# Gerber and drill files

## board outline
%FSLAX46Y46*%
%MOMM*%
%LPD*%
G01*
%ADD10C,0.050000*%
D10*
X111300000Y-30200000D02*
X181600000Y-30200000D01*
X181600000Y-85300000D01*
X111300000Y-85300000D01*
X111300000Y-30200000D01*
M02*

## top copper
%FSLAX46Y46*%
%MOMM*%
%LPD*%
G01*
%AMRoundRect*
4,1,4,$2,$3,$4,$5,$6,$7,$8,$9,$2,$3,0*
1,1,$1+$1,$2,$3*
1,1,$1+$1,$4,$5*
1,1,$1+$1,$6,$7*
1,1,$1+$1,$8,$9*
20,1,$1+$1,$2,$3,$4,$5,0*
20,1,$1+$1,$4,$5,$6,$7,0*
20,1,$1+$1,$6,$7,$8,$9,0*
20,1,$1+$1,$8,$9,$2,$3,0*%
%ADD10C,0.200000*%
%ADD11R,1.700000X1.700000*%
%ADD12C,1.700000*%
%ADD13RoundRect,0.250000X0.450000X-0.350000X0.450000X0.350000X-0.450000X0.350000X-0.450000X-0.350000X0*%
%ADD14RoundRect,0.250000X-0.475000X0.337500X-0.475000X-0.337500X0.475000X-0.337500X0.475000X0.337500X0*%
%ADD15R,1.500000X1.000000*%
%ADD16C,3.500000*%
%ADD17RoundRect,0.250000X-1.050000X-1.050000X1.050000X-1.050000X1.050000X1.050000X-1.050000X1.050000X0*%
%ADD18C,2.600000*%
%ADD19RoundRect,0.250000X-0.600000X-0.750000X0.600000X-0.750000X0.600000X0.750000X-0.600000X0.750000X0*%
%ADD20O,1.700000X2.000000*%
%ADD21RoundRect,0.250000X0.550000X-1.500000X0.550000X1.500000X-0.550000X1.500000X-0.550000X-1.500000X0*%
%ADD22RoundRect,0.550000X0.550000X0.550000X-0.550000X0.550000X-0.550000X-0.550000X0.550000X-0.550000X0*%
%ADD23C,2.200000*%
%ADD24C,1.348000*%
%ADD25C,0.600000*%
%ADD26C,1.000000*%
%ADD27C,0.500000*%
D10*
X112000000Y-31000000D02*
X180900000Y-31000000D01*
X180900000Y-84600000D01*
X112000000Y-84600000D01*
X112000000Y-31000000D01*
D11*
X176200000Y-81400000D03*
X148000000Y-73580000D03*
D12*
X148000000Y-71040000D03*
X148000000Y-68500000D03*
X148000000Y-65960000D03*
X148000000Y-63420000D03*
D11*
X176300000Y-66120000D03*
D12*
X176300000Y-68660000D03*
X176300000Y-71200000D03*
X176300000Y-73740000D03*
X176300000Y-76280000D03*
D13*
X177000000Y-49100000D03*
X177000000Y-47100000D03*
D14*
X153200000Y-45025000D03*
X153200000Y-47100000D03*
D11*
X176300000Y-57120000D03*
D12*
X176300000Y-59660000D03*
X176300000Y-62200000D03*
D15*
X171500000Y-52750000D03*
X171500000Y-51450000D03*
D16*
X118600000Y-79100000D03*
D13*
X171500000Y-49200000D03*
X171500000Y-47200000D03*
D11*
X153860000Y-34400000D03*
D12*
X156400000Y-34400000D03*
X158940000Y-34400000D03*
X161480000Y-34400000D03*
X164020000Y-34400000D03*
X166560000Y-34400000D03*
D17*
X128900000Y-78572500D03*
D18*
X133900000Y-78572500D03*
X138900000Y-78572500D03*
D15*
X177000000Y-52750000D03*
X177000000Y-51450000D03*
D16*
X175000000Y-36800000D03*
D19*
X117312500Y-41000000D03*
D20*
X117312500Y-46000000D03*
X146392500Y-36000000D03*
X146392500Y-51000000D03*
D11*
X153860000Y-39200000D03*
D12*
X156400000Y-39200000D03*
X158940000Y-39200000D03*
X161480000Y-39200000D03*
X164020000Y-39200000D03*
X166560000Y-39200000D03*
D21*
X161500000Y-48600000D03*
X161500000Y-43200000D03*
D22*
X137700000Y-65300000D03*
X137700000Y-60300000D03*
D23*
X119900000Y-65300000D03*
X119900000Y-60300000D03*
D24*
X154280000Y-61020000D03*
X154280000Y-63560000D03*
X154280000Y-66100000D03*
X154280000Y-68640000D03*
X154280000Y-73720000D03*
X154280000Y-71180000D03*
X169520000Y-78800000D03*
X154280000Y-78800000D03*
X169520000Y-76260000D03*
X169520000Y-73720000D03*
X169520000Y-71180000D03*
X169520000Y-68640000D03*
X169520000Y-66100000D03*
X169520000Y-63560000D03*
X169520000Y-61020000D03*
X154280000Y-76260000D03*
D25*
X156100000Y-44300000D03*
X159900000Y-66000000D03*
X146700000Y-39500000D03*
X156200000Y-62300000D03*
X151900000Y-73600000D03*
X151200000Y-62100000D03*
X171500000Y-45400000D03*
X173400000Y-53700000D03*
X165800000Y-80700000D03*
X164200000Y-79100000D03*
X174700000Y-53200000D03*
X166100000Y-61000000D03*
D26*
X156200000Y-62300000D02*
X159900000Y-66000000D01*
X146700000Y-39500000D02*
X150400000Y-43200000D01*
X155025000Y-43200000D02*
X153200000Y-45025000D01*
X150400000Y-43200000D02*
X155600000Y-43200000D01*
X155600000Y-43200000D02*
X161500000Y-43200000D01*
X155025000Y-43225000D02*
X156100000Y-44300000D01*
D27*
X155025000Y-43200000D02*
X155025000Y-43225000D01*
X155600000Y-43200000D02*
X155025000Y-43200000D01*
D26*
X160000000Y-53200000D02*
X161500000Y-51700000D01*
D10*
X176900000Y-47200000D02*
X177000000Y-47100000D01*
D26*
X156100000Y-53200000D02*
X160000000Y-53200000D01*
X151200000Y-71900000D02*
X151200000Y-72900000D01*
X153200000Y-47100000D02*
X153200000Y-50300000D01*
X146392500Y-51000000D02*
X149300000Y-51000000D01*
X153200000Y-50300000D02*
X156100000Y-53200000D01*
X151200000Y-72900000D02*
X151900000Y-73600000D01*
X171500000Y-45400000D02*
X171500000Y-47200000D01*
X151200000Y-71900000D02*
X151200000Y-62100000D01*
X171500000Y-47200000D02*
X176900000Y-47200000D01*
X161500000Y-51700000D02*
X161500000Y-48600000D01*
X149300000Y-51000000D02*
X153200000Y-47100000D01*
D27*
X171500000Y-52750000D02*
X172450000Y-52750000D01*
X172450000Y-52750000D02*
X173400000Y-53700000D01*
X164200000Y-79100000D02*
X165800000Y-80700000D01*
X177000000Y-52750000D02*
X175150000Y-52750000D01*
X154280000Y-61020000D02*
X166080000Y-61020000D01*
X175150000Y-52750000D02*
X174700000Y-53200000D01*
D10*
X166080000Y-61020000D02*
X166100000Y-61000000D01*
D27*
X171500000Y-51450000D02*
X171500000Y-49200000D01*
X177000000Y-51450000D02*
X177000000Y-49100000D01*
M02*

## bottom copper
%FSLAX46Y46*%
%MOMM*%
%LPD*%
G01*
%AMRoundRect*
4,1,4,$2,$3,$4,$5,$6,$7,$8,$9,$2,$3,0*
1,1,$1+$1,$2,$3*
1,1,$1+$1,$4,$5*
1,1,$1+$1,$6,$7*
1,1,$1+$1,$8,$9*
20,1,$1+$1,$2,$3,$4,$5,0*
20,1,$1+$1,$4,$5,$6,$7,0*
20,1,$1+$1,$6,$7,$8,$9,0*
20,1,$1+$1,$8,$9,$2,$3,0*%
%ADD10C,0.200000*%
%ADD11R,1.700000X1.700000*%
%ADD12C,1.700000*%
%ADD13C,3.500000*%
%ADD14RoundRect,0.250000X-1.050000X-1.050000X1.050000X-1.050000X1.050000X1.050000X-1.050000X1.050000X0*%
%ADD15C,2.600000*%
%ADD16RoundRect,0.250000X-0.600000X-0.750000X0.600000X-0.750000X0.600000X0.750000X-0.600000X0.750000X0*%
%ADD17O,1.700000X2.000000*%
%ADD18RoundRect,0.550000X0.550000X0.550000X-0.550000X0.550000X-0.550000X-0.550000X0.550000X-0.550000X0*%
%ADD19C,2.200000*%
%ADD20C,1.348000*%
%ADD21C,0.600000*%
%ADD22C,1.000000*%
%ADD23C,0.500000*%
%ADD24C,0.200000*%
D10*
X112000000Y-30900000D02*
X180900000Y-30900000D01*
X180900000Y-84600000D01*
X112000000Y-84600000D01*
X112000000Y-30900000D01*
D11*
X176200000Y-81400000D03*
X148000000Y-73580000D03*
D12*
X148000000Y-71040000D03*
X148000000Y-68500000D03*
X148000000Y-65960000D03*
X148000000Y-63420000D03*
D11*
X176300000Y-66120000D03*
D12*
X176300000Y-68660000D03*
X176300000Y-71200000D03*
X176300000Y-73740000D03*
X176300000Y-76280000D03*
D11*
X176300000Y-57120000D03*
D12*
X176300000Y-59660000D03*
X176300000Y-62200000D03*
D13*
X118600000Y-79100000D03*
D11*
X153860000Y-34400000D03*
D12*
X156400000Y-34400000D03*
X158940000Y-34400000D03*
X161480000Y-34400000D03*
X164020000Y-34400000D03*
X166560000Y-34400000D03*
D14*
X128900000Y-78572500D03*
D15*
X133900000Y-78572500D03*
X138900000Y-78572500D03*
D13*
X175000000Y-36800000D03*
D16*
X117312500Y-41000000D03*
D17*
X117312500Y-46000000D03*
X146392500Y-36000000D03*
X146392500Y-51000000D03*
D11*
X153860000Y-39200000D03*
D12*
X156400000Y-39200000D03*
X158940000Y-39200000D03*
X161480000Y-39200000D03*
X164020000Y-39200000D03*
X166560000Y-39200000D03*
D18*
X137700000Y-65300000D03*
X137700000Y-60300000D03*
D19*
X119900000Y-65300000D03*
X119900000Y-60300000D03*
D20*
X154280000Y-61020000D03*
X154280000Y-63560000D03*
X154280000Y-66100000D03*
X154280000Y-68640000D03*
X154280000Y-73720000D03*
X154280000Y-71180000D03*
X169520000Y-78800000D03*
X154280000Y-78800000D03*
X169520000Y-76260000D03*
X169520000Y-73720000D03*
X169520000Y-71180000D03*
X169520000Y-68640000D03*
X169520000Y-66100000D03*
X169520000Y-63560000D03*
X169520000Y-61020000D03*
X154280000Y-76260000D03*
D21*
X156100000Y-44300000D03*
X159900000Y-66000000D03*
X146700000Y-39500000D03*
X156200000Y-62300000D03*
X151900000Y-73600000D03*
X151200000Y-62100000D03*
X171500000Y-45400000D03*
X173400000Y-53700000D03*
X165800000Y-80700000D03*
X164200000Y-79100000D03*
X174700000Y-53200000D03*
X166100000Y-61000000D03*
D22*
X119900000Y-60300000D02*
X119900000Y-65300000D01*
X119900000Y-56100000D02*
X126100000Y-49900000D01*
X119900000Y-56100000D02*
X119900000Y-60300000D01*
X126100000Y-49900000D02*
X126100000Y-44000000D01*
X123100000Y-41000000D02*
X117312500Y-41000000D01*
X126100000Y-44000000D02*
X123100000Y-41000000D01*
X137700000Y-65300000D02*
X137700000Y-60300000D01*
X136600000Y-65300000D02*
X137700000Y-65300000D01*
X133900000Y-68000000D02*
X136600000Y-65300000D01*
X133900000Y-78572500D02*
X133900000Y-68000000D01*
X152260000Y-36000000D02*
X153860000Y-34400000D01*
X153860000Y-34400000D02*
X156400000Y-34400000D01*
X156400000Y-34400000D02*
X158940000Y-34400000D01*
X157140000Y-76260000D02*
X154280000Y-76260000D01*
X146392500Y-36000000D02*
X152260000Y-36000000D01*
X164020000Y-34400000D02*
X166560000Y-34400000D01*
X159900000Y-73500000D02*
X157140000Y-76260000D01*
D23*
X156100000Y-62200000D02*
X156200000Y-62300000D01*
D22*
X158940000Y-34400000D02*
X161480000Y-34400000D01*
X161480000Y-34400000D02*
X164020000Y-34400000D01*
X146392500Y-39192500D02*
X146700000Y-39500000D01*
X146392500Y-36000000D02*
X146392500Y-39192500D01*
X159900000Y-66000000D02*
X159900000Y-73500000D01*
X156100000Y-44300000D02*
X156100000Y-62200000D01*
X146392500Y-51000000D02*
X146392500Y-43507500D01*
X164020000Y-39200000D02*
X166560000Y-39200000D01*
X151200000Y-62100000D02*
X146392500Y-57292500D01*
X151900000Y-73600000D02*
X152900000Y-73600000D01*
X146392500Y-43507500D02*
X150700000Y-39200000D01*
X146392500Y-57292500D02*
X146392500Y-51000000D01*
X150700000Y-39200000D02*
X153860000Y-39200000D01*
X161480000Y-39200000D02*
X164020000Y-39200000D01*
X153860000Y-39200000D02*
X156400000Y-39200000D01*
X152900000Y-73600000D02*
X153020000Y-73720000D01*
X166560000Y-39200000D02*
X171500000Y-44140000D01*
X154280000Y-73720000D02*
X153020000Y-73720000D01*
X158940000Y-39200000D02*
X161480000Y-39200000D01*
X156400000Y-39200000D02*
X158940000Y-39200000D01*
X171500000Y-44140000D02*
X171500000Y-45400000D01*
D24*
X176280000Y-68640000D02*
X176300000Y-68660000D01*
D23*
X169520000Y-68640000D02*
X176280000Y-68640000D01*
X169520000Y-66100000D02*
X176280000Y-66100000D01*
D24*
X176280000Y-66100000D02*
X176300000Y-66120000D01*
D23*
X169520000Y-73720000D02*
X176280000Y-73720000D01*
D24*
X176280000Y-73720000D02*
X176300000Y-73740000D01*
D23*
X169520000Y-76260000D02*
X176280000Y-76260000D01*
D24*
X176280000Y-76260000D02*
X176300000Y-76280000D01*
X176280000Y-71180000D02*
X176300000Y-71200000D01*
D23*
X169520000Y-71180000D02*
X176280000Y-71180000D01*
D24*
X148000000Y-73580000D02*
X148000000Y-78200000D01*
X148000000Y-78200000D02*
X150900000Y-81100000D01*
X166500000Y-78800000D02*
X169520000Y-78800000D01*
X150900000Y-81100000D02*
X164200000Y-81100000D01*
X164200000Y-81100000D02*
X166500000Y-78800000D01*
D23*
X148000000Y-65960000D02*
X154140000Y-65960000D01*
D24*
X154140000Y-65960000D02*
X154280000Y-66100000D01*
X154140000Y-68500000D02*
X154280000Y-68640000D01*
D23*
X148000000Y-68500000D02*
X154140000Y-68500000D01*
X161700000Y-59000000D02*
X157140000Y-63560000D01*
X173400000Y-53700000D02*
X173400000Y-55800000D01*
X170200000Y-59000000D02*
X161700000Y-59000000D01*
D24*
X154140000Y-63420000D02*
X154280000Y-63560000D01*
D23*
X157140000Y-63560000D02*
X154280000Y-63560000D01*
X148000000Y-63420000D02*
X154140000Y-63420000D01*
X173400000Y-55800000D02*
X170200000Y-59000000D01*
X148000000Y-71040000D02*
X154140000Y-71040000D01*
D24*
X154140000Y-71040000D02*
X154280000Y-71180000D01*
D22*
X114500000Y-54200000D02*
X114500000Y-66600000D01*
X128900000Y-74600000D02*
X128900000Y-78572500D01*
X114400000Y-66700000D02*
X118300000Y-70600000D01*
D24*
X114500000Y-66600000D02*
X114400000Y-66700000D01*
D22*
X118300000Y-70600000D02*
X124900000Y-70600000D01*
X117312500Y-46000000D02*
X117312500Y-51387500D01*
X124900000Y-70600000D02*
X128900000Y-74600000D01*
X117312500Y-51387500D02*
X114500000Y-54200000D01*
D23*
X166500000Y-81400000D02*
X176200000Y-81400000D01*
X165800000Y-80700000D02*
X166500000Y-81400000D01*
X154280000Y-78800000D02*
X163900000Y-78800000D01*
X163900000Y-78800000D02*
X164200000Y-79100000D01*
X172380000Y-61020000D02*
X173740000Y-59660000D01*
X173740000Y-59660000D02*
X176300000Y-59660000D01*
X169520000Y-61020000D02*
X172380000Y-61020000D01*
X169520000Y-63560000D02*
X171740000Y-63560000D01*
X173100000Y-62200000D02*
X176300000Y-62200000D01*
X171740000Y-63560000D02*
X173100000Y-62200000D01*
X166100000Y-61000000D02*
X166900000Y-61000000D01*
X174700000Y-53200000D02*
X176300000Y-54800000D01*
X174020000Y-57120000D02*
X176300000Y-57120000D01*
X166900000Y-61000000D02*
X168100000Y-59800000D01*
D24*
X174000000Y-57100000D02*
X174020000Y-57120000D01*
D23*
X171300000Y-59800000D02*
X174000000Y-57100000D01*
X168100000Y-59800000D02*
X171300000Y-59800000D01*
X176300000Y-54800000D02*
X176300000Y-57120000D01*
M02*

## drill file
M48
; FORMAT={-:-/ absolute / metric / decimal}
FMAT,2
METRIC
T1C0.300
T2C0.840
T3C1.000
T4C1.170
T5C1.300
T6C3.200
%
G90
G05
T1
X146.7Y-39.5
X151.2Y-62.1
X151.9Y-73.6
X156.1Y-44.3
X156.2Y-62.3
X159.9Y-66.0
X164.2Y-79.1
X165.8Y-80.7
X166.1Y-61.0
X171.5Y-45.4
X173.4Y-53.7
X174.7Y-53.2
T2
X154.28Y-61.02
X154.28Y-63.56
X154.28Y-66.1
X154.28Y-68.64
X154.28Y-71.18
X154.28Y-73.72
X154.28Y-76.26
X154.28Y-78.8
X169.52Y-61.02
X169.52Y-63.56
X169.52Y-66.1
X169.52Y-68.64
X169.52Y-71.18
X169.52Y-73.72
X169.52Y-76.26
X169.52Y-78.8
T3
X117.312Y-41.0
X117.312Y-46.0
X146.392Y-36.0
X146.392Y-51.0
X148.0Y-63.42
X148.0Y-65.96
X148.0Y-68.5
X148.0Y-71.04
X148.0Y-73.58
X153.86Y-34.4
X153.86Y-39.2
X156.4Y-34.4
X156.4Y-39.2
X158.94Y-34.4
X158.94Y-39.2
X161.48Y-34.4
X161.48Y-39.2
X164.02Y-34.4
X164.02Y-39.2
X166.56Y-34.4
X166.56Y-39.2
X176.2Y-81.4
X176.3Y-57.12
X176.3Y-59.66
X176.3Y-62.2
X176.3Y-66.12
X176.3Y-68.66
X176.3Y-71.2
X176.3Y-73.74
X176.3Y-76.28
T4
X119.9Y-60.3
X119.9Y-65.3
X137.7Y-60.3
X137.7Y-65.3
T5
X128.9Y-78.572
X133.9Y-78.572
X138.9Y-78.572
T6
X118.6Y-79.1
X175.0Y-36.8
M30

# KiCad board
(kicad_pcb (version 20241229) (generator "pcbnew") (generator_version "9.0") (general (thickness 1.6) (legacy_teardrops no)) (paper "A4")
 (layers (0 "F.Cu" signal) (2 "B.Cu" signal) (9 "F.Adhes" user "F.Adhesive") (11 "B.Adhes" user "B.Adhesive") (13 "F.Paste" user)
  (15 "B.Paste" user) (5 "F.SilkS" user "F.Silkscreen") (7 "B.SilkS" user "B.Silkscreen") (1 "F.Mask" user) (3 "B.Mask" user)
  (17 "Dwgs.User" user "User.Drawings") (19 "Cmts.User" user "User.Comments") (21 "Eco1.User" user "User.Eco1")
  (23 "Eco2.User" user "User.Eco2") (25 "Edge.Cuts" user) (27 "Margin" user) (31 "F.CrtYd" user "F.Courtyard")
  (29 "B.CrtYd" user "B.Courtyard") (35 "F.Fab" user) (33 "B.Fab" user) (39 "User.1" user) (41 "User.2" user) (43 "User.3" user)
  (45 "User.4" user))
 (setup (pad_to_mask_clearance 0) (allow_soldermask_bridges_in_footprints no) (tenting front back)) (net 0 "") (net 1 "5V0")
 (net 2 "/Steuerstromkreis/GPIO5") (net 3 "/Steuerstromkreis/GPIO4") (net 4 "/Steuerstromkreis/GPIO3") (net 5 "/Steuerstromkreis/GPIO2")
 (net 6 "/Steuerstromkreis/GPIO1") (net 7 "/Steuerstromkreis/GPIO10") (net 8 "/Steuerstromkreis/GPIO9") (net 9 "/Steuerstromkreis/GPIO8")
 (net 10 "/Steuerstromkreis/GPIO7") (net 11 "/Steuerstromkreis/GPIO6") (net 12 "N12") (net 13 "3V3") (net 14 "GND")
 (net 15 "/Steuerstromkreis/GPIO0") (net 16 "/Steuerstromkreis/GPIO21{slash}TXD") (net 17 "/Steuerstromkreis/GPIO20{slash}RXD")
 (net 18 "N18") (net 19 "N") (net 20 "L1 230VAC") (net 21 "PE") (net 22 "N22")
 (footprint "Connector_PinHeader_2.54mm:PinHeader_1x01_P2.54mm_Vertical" (layer "F.Cu") (at 176.2 81.4)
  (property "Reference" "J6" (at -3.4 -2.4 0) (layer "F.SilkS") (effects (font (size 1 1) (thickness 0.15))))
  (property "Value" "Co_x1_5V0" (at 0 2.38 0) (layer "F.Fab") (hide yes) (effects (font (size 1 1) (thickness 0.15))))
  (pad "1" thru_hole rect (at 0 0) (size 1.7 1.7) (drill 1) (layers "*.Cu" "*.Mask") (remove_unused_layers no) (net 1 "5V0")))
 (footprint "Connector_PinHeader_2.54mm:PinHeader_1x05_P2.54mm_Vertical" (layer "F.Cu") (at 148 73.58 180)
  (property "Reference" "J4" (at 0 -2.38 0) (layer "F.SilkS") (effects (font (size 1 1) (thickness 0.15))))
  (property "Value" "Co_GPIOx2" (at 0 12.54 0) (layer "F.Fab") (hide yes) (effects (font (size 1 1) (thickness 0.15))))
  (pad "1" thru_hole rect (at 0 0 180) (size 1.7 1.7) (drill 1) (layers "*.Cu" "*.Mask") (remove_unused_layers no)
   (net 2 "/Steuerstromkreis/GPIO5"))
  (pad "2" thru_hole circle (at 0 2.54 180) (size 1.7 1.7) (drill 1) (layers "*.Cu" "*.Mask") (remove_unused_layers no)
   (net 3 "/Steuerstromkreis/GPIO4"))
  (pad "3" thru_hole circle (at 0 5.08 180) (size 1.7 1.7) (drill 1) (layers "*.Cu" "*.Mask") (remove_unused_layers no)
   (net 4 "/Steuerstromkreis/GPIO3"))
  (pad "4" thru_hole circle (at 0 7.62 180) (size 1.7 1.7) (drill 1) (layers "*.Cu" "*.Mask") (remove_unused_layers no)
   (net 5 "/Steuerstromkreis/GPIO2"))
  (pad "5" thru_hole circle (at 0 10.16 180) (size 1.7 1.7) (drill 1) (layers "*.Cu" "*.Mask") (remove_unused_layers no)
   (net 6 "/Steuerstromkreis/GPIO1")))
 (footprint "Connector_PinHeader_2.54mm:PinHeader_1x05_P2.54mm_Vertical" (layer "F.Cu") (at 176.3 66.12)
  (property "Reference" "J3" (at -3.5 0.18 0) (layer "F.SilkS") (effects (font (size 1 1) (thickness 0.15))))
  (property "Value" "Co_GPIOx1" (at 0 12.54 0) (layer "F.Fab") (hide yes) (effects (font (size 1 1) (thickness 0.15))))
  (pad "1" thru_hole rect (at 0 0) (size 1.7 1.7) (drill 1) (layers "*.Cu" "*.Mask") (remove_unused_layers no)
   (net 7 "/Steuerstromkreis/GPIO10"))
  (pad "2" thru_hole circle (at 0 2.54) (size 1.7 1.7) (drill 1) (layers "*.Cu" "*.Mask") (remove_unused_layers no)
   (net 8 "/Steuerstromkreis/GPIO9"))
  (pad "3" thru_hole circle (at 0 5.08) (size 1.7 1.7) (drill 1) (layers "*.Cu" "*.Mask") (remove_unused_layers no)
   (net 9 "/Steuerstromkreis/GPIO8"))
  (pad "4" thru_hole circle (at 0 7.62) (size 1.7 1.7) (drill 1) (layers "*.Cu" "*.Mask") (remove_unused_layers no)
   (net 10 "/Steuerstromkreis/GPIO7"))
  (pad "5" thru_hole circle (at 0 10.16) (size 1.7 1.7) (drill 1) (layers "*.Cu" "*.Mask") (remove_unused_layers no)
   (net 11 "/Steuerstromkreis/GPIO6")))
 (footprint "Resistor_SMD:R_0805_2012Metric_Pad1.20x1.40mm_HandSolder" (layer "F.Cu") (at 177 48.1 90)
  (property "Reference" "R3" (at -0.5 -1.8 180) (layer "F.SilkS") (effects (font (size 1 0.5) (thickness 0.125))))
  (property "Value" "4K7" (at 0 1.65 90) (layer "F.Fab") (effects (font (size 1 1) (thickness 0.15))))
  (pad "1" smd roundrect (at -1 0 90) (size 1.2 1.4) (layers "F.Cu" "F.Mask" "F.Paste") (roundrect_rratio 0.208333) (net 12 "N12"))
  (pad "2" smd roundrect (at 1 0 90) (size 1.2 1.4) (layers "F.Cu" "F.Mask" "F.Paste") (roundrect_rratio 0.208333) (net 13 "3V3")))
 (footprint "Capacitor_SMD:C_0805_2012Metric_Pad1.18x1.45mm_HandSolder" (layer "F.Cu") (at 153.2 46.0625 -90)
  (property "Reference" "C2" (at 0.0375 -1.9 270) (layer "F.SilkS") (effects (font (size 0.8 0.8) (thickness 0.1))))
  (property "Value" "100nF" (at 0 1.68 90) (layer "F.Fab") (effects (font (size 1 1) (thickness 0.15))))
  (pad "1" smd roundrect (at -1.0375 0 270) (size 1.175 1.45) (layers "F.Cu" "F.Mask" "F.Paste") (roundrect_rratio 0.212766) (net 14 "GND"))
  (pad "2" smd roundrect (at 1.0375 0 270) (size 1.175 1.45) (layers "F.Cu" "F.Mask" "F.Paste") (roundrect_rratio 0.212766) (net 13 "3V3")))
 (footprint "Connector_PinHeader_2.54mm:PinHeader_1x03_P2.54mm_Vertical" (layer "F.Cu") (at 176.3 57.12)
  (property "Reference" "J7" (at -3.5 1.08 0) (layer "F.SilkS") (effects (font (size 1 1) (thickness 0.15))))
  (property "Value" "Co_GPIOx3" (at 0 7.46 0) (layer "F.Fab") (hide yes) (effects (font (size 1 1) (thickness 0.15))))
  (pad "1" thru_hole rect (at 0 0) (size 1.7 1.7) (drill 1) (layers "*.Cu" "*.Mask") (remove_unused_layers no)
   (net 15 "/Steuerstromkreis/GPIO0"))
  (pad "2" thru_hole circle (at 0 2.54) (size 1.7 1.7) (drill 1) (layers "*.Cu" "*.Mask") (remove_unused_layers no)
   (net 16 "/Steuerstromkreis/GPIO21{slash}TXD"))
  (pad "3" thru_hole circle (at 0 5.08) (size 1.7 1.7) (drill 1) (layers "*.Cu" "*.Mask") (remove_unused_layers no)
   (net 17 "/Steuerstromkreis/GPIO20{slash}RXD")))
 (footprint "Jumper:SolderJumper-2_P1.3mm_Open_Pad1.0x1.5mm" (layer "F.Cu") (at 171.5 52.1 90)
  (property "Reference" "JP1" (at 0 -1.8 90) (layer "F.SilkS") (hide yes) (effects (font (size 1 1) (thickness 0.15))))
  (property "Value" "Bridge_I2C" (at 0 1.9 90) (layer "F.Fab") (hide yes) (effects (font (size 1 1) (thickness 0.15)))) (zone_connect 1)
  (pad "1" smd rect (at -0.65 0 90) (size 1 1.5) (layers "F.Cu" "F.Mask") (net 6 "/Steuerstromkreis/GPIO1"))
  (pad "2" smd rect (at 0.65 0 90) (size 1 1.5) (layers "F.Cu" "F.Mask") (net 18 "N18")))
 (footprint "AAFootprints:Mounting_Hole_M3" (layer "F.Cu") (at 118.6 79.1)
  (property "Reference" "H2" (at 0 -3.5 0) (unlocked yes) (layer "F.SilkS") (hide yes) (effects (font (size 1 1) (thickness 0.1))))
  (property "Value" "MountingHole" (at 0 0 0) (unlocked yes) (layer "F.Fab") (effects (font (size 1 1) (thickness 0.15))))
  (pad "" np_thru_hole circle (at 0 0) (size 3.5 3.5) (drill 3.2) (layers "*.Cu" "*.Mask")))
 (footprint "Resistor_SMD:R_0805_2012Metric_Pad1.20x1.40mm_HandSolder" (layer "F.Cu") (at 171.5 48.2 90)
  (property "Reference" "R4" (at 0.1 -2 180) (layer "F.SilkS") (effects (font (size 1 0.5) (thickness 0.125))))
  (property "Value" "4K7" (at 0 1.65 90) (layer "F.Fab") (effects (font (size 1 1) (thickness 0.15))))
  (pad "1" smd roundrect (at -1 0 90) (size 1.2 1.4) (layers "F.Cu" "F.Mask" "F.Paste") (roundrect_rratio 0.208333) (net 18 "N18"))
  (pad "2" smd roundrect (at 1 0 90) (size 1.2 1.4) (layers "F.Cu" "F.Mask" "F.Paste") (roundrect_rratio 0.208333) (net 13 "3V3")))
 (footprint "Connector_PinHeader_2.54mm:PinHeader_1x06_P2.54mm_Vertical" (layer "F.Cu") (at 153.86 34.4 90)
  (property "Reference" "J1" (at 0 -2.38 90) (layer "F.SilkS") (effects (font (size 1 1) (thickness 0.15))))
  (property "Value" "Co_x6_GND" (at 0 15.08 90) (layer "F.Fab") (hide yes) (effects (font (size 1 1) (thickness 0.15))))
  (pad "1" thru_hole rect (at 0 0 90) (size 1.7 1.7) (drill 1) (layers "*.Cu" "*.Mask") (remove_unused_layers no) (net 14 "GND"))
  (pad "2" thru_hole circle (at 0 2.54 90) (size 1.7 1.7) (drill 1) (layers "*.Cu" "*.Mask") (remove_unused_layers no) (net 14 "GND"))
  (pad "3" thru_hole circle (at 0 5.08 90) (size 1.7 1.7) (drill 1) (layers "*.Cu" "*.Mask") (remove_unused_layers no) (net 14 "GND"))
  (pad "4" thru_hole circle (at 0 7.62 90) (size 1.7 1.7) (drill 1) (layers "*.Cu" "*.Mask") (remove_unused_layers no) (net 14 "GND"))
  (pad "5" thru_hole circle (at 0 10.16 90) (size 1.7 1.7) (drill 1) (layers "*.Cu" "*.Mask") (remove_unused_layers no) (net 14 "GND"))
  (pad "6" thru_hole circle (at 0 12.7 90) (size 1.7 1.7) (drill 1) (layers "*.Cu" "*.Mask") (remove_unused_layers no) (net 14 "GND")))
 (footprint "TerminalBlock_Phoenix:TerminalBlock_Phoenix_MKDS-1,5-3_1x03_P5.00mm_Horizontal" (layer "F.Cu") (at 128.9 78.5725)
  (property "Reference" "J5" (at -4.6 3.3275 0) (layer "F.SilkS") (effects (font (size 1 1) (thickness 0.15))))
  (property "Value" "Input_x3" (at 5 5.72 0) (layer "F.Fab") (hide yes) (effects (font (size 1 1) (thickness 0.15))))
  (pad "1" thru_hole roundrect (at 0 0) (size 2.6 2.6) (drill 1.3) (layers "*.Cu" "*.Mask") (remove_unused_layers no)
   (roundrect_rratio 0.096154) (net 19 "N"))
  (pad "2" thru_hole circle (at 5 0) (size 2.6 2.6) (drill 1.3) (layers "*.Cu" "*.Mask") (remove_unused_layers no) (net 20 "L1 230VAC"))
  (pad "3" thru_hole circle (at 10 0) (size 2.6 2.6) (drill 1.3) (layers "*.Cu" "*.Mask") (remove_unused_layers no) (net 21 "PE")))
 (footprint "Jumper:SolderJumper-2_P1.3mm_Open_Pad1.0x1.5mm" (layer "F.Cu") (at 177 52.1 90)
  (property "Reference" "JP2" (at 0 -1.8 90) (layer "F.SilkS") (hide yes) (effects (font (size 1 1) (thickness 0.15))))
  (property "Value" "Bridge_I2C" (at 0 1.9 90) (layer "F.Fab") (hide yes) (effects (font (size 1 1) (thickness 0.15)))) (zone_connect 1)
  (pad "1" smd rect (at -0.65 0 90) (size 1 1.5) (layers "F.Cu" "F.Mask") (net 15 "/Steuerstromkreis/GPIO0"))
  (pad "2" smd rect (at 0.65 0 90) (size 1 1.5) (layers "F.Cu" "F.Mask") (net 12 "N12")))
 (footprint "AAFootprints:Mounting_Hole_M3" (layer "F.Cu") (at 175 36.8)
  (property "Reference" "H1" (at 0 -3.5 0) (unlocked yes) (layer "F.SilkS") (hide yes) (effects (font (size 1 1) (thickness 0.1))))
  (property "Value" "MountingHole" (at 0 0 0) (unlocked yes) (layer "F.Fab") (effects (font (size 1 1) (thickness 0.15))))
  (pad "" np_thru_hole circle (at 0 0) (size 3.5 3.5) (drill 3.2) (layers "*.Cu" "*.Mask")))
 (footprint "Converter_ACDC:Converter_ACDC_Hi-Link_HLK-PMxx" (layer "F.Cu") (at 117.3125 41)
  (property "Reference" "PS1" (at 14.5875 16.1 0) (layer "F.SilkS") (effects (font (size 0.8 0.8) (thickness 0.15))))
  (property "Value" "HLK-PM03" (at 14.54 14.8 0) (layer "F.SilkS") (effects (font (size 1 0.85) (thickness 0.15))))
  (pad "1" thru_hole roundrect (at 0 0) (size 1.7 2) (drill 1) (layers "*.Cu" "*.Mask") (remove_unused_layers no)
   (roundrect_rratio 0.147059) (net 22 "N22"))
  (pad "2" thru_hole oval (at 0 5) (size 1.7 2) (drill 1) (layers "*.Cu" "*.Mask") (remove_unused_layers no) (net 19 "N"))
  (pad "3" thru_hole oval (at 29.08 -5) (size 1.7 2) (drill 1) (layers "*.Cu" "*.Mask") (remove_unused_layers no) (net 14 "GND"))
  (pad "4" thru_hole oval (at 29.08 10) (size 1.7 2) (drill 1) (layers "*.Cu" "*.Mask") (remove_unused_layers no) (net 13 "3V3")))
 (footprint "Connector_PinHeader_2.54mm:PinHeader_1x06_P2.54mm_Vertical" (layer "F.Cu") (at 153.86 39.2 90)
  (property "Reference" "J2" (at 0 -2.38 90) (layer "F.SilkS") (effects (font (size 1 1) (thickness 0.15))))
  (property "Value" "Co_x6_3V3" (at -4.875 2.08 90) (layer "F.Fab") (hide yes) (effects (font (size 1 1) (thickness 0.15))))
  (pad "1" thru_hole rect (at 0 0 90) (size 1.7 1.7) (drill 1) (layers "*.Cu" "*.Mask") (remove_unused_layers no) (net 13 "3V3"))
  (pad "2" thru_hole circle (at 0 2.54 90) (size 1.7 1.7) (drill 1) (layers "*.Cu" "*.Mask") (remove_unused_layers no) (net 13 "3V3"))
  (pad "3" thru_hole circle (at 0 5.08 90) (size 1.7 1.7) (drill 1) (layers "*.Cu" "*.Mask") (remove_unused_layers no) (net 13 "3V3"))
  (pad "4" thru_hole circle (at 0 7.62 90) (size 1.7 1.7) (drill 1) (layers "*.Cu" "*.Mask") (remove_unused_layers no) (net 13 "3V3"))
  (pad "5" thru_hole circle (at 0 10.16 90) (size 1.7 1.7) (drill 1) (layers "*.Cu" "*.Mask") (remove_unused_layers no) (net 13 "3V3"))
  (pad "6" thru_hole circle (at 0 12.7 90) (size 1.7 1.7) (drill 1) (layers "*.Cu" "*.Mask") (remove_unused_layers no) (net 13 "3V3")))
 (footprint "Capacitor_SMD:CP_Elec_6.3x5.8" (layer "F.Cu") (at 161.5 45.9 90)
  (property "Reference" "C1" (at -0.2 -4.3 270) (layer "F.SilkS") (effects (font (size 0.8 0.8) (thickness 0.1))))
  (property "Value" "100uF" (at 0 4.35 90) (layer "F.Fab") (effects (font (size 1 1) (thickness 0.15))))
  (pad "1" smd roundrect (at -2.7 0 90) (size 3.5 1.6) (layers "F.Cu" "F.Mask" "F.Paste") (roundrect_rratio 0.15625) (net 13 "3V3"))
  (pad "2" smd roundrect (at 2.7 0 90) (size 3.5 1.6) (layers "F.Cu" "F.Mask" "F.Paste") (roundrect_rratio 0.15625) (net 14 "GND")))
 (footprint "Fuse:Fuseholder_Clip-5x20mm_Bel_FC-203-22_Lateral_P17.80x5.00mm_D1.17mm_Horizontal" (layer "F.Cu") (at 137.7 65.3 180)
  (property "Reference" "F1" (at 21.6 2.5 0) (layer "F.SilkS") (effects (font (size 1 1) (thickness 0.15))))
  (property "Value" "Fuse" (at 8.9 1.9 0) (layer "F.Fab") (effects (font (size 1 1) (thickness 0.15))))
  (pad "1" thru_hole roundrect (at 0 0 180) (size 2.2 2.2) (drill 1.17) (layers "*.Cu" "*.Mask") (remove_unused_layers no)
   (roundrect_rratio 0.25) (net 20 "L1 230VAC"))
  (pad "1" thru_hole roundrect (at 0 5 180) (size 2.2 2.2) (drill 1.17) (layers "*.Cu" "*.Mask") (remove_unused_layers no)
   (roundrect_rratio 0.25) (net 20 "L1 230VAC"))
  (pad "2" thru_hole circle (at 17.8 0 180) (size 2.2 2.2) (drill 1.17) (layers "*.Cu" "*.Mask") (remove_unused_layers no) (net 22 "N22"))
  (pad "2" thru_hole circle (at 17.8 5 180) (size 2.2 2.2) (drill 1.17) (layers "*.Cu" "*.Mask") (remove_unused_layers no) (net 22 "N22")))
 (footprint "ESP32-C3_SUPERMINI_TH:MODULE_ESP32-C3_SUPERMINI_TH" (layer "F.Cu") (at 161.9 68.9 180)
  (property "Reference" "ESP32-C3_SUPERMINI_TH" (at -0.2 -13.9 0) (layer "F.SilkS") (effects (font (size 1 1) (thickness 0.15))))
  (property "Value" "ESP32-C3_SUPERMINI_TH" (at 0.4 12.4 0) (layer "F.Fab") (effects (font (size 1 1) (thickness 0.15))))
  (pad "0" thru_hole circle (at 7.62 7.88 180) (size 1.348 1.348) (drill 0.84) (layers "*.Cu" "*.Mask") (remove_unused_layers no)
   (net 15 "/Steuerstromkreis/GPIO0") (solder_mask_margin 0.102))
  (pad "1" thru_hole circle (at 7.62 5.34 180) (size 1.348 1.348) (drill 0.84) (layers "*.Cu" "*.Mask") (remove_unused_layers no)
   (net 6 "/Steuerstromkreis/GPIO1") (solder_mask_margin 0.102))
  (pad "2" thru_hole circle (at 7.62 2.8 180) (size 1.348 1.348) (drill 0.84) (layers "*.Cu" "*.Mask") (remove_unused_layers no)
   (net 5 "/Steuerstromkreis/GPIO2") (solder_mask_margin 0.102))
  (pad "3" thru_hole circle (at 7.62 0.26 180) (size 1.348 1.348) (drill 0.84) (layers "*.Cu" "*.Mask") (remove_unused_layers no)
   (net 4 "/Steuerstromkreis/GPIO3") (solder_mask_margin 0.102))
  (pad "3.3" thru_hole circle (at 7.62 -4.82 180) (size 1.348 1.348) (drill 0.84) (layers "*.Cu" "*.Mask") (remove_unused_layers no)
   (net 13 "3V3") (solder_mask_margin 0.102))
  (pad "4" thru_hole circle (at 7.62 -2.28 180) (size 1.348 1.348) (drill 0.84) (layers "*.Cu" "*.Mask") (remove_unused_layers no)
   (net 3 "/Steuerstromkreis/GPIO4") (solder_mask_margin 0.102))
  (pad "5" thru_hole circle (at -7.62 -9.9 180) (size 1.348 1.348) (drill 0.84) (layers "*.Cu" "*.Mask") (remove_unused_layers no)
   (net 2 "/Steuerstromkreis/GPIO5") (solder_mask_margin 0.102))
  (pad "5V" thru_hole circle (at 7.62 -9.9 180) (size 1.348 1.348) (drill 0.84) (layers "*.Cu" "*.Mask") (remove_unused_layers no)
   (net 1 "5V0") (solder_mask_margin 0.102))
  (pad "6" thru_hole circle (at -7.62 -7.36 180) (size 1.348 1.348) (drill 0.84) (layers "*.Cu" "*.Mask") (remove_unused_layers no)
   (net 11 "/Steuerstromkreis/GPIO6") (solder_mask_margin 0.102))
  (pad "7" thru_hole circle (at -7.62 -4.82 180) (size 1.348 1.348) (drill 0.84) (layers "*.Cu" "*.Mask") (remove_unused_layers no)
   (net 10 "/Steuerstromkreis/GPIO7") (solder_mask_margin 0.102))
  (pad "8" thru_hole circle (at -7.62 -2.28 180) (size 1.348 1.348) (drill 0.84) (layers "*.Cu" "*.Mask") (remove_unused_layers no)
   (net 9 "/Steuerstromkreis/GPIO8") (solder_mask_margin 0.102))
  (pad "9" thru_hole circle (at -7.62 0.26 180) (size 1.348 1.348) (drill 0.84) (layers "*.Cu" "*.Mask") (remove_unused_layers no)
   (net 8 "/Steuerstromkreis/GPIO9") (solder_mask_margin 0.102))
  (pad "10" thru_hole circle (at -7.62 2.8 180) (size 1.348 1.348) (drill 0.84) (layers "*.Cu" "*.Mask") (remove_unused_layers no)
   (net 7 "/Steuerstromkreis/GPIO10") (solder_mask_margin 0.102))
  (pad "20" thru_hole circle (at -7.62 5.34 180) (size 1.348 1.348) (drill 0.84) (layers "*.Cu" "*.Mask") (remove_unused_layers no)
   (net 17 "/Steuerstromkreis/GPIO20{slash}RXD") (solder_mask_margin 0.102))
  (pad "21" thru_hole circle (at -7.62 7.88 180) (size 1.348 1.348) (drill 0.84) (layers "*.Cu" "*.Mask") (remove_unused_layers no)
   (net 16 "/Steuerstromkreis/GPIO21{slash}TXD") (solder_mask_margin 0.102))
  (pad "G" thru_hole circle (at 7.62 -7.36 180) (size 1.348 1.348) (drill 0.84) (layers "*.Cu" "*.Mask") (remove_unused_layers no)
   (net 14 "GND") (solder_mask_margin 0.102)))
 (gr_rect (start 112 31) (end 180.9 84.6) (stroke (width 0.2) (type default)) (fill no) (layer "F.Cu") (net 13))
 (gr_rect (start 112 30.9) (end 180.9 84.6) (stroke (width 0.2) (type default)) (fill no) (layer "B.Cu"))
 (gr_rect (start 111.3 30.2) (end 181.6 85.3) (stroke (width 0.05) (type default)) (fill no) (layer "Edge.Cuts"))
 (segment (start 119.9 60.3) (end 119.9 65.3) (width 1) (layer "B.Cu") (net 22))
 (segment (start 119.9 56.1) (end 126.1 49.9) (width 1) (layer "B.Cu") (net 22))
 (segment (start 119.9 56.1) (end 119.9 60.3) (width 1) (layer "B.Cu") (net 22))
 (segment (start 126.1 49.9) (end 126.1 44) (width 1) (layer "B.Cu") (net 22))
 (segment (start 123.1 41) (end 117.3125 41) (width 1) (layer "B.Cu") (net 22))
 (segment (start 126.1 44) (end 123.1 41) (width 1) (layer "B.Cu") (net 22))
 (segment (start 137.7 65.3) (end 137.7 60.3) (width 1) (layer "B.Cu") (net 20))
 (segment (start 136.6 65.3) (end 137.7 65.3) (width 1) (layer "B.Cu") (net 20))
 (segment (start 133.9 68) (end 136.6 65.3) (width 1) (layer "B.Cu") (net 20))
 (segment (start 133.9 78.5725) (end 133.9 68) (width 1) (layer "B.Cu") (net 20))
 (segment (start 156.2 62.3) (end 159.9 66) (width 1) (layer "F.Cu") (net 14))
 (segment (start 146.7 39.5) (end 150.4 43.2) (width 1) (layer "F.Cu") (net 14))
 (segment (start 155.025 43.2) (end 153.2 45.025) (width 1) (layer "F.Cu") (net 14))
 (segment (start 150.4 43.2) (end 155.6 43.2) (width 1) (layer "F.Cu") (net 14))
 (segment (start 155.6 43.2) (end 161.5 43.2) (width 1) (layer "F.Cu") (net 14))
 (segment (start 155.025 43.225) (end 156.1 44.3) (width 1) (layer "F.Cu") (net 14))
 (segment (start 155.025 43.2) (end 155.025 43.225) (width 0.5) (layer "F.Cu") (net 14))
 (segment (start 155.6 43.2) (end 155.025 43.2) (width 0.5) (layer "F.Cu") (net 14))
 (via (at 156.1 44.3) (size 0.6) (drill 0.3) (layers "F.Cu" "B.Cu") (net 14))
 (via (at 159.9 66) (size 0.6) (drill 0.3) (layers "F.Cu" "B.Cu") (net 14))
 (via (at 146.7 39.5) (size 0.6) (drill 0.3) (layers "F.Cu" "B.Cu") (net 14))
 (via (at 156.2 62.3) (size 0.6) (drill 0.3) (layers "F.Cu" "B.Cu") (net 14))
 (segment (start 152.26 36) (end 153.86 34.4) (width 1) (layer "B.Cu") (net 14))
 (segment (start 153.86 34.4) (end 156.4 34.4) (width 1) (layer "B.Cu") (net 14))
 (segment (start 156.4 34.4) (end 158.94 34.4) (width 1) (layer "B.Cu") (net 14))
 (segment (start 157.14 76.26) (end 154.28 76.26) (width 1) (layer "B.Cu") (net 14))
 (segment (start 146.3925 36) (end 152.26 36) (width 1) (layer "B.Cu") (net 14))
 (segment (start 164.02 34.4) (end 166.56 34.4) (width 1) (layer "B.Cu") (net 14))
 (segment (start 159.9 73.5) (end 157.14 76.26) (width 1) (layer "B.Cu") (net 14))
 (segment (start 156.1 62.2) (end 156.2 62.3) (width 0.5) (layer "B.Cu") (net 14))
 (segment (start 158.94 34.4) (end 161.48 34.4) (width 1) (layer "B.Cu") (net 14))
 (segment (start 161.48 34.4) (end 164.02 34.4) (width 1) (layer "B.Cu") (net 14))
 (segment (start 146.3925 39.1925) (end 146.7 39.5) (width 1) (layer "B.Cu") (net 14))
 (segment (start 146.3925 36) (end 146.3925 39.1925) (width 1) (layer "B.Cu") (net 14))
 (segment (start 159.9 66) (end 159.9 73.5) (width 1) (layer "B.Cu") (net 14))
 (segment (start 156.1 44.3) (end 156.1 62.2) (width 1) (layer "B.Cu") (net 14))
 (segment (start 160 53.2) (end 161.5 51.7) (width 1) (layer "F.Cu") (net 13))
 (segment (start 176.9 47.2) (end 177 47.1) (width 0.2) (layer "F.Cu") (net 13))
 (segment (start 156.1 53.2) (end 160 53.2) (width 1) (layer "F.Cu") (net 13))
 (segment (start 151.2 71.9) (end 151.2 72.9) (width 1) (layer "F.Cu") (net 13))
 (segment (start 153.2 47.1) (end 153.2 50.3) (width 1) (layer "F.Cu") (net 13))
 (segment (start 146.3925 51) (end 149.3 51) (width 1) (layer "F.Cu") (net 13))
 (segment (start 153.2 50.3) (end 156.1 53.2) (width 1) (layer "F.Cu") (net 13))
 (segment (start 151.2 72.9) (end 151.9 73.6) (width 1) (layer "F.Cu") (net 13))
 (segment (start 171.5 45.4) (end 171.5 47.2) (width 1) (layer "F.Cu") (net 13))
 (segment (start 151.2 71.9) (end 151.2 62.1) (width 1) (layer "F.Cu") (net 13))
 (segment (start 171.5 47.2) (end 176.9 47.2) (width 1) (layer "F.Cu") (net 13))
 (segment (start 161.5 51.7) (end 161.5 48.6) (width 1) (layer "F.Cu") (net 13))
 (segment (start 149.3 51) (end 153.2 47.1) (width 1) (layer "F.Cu") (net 13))
 (via (at 151.9 73.6) (size 0.6) (drill 0.3) (layers "F.Cu" "B.Cu") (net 13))
 (via (at 151.2 62.1) (size 0.6) (drill 0.3) (layers "F.Cu" "B.Cu") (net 13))
 (via (at 171.5 45.4) (size 0.6) (drill 0.3) (layers "F.Cu" "B.Cu") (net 13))
 (segment (start 146.3925 51) (end 146.3925 43.5075) (width 1) (layer "B.Cu") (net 13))
 (segment (start 164.02 39.2) (end 166.56 39.2) (width 1) (layer "B.Cu") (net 13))
 (segment (start 151.2 62.1) (end 146.3925 57.2925) (width 1) (layer "B.Cu") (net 13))
 (segment (start 151.9 73.6) (end 152.9 73.6) (width 1) (layer "B.Cu") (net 13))
 (segment (start 146.3925 43.5075) (end 150.7 39.2) (width 1) (layer "B.Cu") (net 13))
 (segment (start 146.3925 57.2925) (end 146.3925 51) (width 1) (layer "B.Cu") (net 13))
 (segment (start 150.7 39.2) (end 153.86 39.2) (width 1) (layer "B.Cu") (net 13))
 (segment (start 161.48 39.2) (end 164.02 39.2) (width 1) (layer "B.Cu") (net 13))
 (segment (start 153.86 39.2) (end 156.4 39.2) (width 1) (layer "B.Cu") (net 13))
 (segment (start 152.9 73.6) (end 153.02 73.72) (width 1) (layer "B.Cu") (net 13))
 (segment (start 166.56 39.2) (end 171.5 44.14) (width 1) (layer "B.Cu") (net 13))
 (segment (start 154.28 73.72) (end 153.02 73.72) (width 1) (layer "B.Cu") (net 13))
 (segment (start 158.94 39.2) (end 161.48 39.2) (width 1) (layer "B.Cu") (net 13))
 (segment (start 156.4 39.2) (end 158.94 39.2) (width 1) (layer "B.Cu") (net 13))
 (segment (start 171.5 44.14) (end 171.5 45.4) (width 1) (layer "B.Cu") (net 13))
 (segment (start 176.28 68.64) (end 176.3 68.66) (width 0.2) (layer "B.Cu") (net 8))
 (segment (start 169.52 68.64) (end 176.28 68.64) (width 0.5) (layer "B.Cu") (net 8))
 (segment (start 169.52 66.1) (end 176.28 66.1) (width 0.5) (layer "B.Cu") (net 7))
 (segment (start 176.28 66.1) (end 176.3 66.12) (width 0.2) (layer "B.Cu") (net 7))
 (segment (start 169.52 73.72) (end 176.28 73.72) (width 0.5) (layer "B.Cu") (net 10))
 (segment (start 176.28 73.72) (end 176.3 73.74) (width 0.2) (layer "B.Cu") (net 10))
 (segment (start 169.52 76.26) (end 176.28 76.26) (width 0.5) (layer "B.Cu") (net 11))
 (segment (start 176.28 76.26) (end 176.3 76.28) (width 0.2) (layer "B.Cu") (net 11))
 (segment (start 176.28 71.18) (end 176.3 71.2) (width 0.2) (layer "B.Cu") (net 9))
 (segment (start 169.52 71.18) (end 176.28 71.18) (width 0.5) (layer "B.Cu") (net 9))
 (segment (start 148 73.58) (end 148 78.2) (width 0.2) (layer "B.Cu") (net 2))
 (segment (start 148 78.2) (end 150.9 81.1) (width 0.2) (layer "B.Cu") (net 2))
 (segment (start 166.5 78.8) (end 169.52 78.8) (width 0.2) (layer "B.Cu") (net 2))
 (segment (start 150.9 81.1) (end 164.2 81.1) (width 0.2) (layer "B.Cu") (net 2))
 (segment (start 164.2 81.1) (end 166.5 78.8) (width 0.2) (layer "B.Cu") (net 2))
 (segment (start 148 65.96) (end 154.14 65.96) (width 0.5) (layer "B.Cu") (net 5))
 (segment (start 154.14 65.96) (end 154.28 66.1) (width 0.2) (layer "B.Cu") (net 5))
 (segment (start 154.14 68.5) (end 154.28 68.64) (width 0.2) (layer "B.Cu") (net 4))
 (segment (start 148 68.5) (end 154.14 68.5) (width 0.5) (layer "B.Cu") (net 4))
 (segment (start 171.5 52.75) (end 172.45 52.75) (width 0.5) (layer "F.Cu") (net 6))
 (segment (start 172.45 52.75) (end 173.4 53.7) (width 0.5) (layer "F.Cu") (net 6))
 (via (at 173.4 53.7) (size 0.6) (drill 0.3) (layers "F.Cu" "B.Cu") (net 6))
 (segment (start 161.7 59) (end 157.14 63.56) (width 0.5) (layer "B.Cu") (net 6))
 (segment (start 173.4 53.7) (end 173.4 55.8) (width 0.5) (layer "B.Cu") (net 6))
 (segment (start 170.2 59) (end 161.7 59) (width 0.5) (layer "B.Cu") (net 6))
 (segment (start 154.14 63.42) (end 154.28 63.56) (width 0.2) (layer "B.Cu") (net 6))
 (segment (start 157.14 63.56) (end 154.28 63.56) (width 0.5) (layer "B.Cu") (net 6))
 (segment (start 148 63.42) (end 154.14 63.42) (width 0.5) (layer "B.Cu") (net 6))
 (segment (start 173.4 55.8) (end 170.2 59) (width 0.5) (layer "B.Cu") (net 6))
 (segment (start 148 71.04) (end 154.14 71.04) (width 0.5) (layer "B.Cu") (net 3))
 (segment (start 154.14 71.04) (end 154.28 71.18) (width 0.2) (layer "B.Cu") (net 3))
 (segment (start 114.5 54.2) (end 114.5 66.6) (width 1) (layer "B.Cu") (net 19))
 (segment (start 128.9 74.6) (end 128.9 78.5725) (width 1) (layer "B.Cu") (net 19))
 (segment (start 114.4 66.7) (end 118.3 70.6) (width 1) (layer "B.Cu") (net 19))
 (segment (start 114.5 66.6) (end 114.4 66.7) (width 0.2) (layer "B.Cu") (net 19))
 (segment (start 118.3 70.6) (end 124.9 70.6) (width 1) (layer "B.Cu") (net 19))
 (segment (start 117.3125 46) (end 117.3125 51.3875) (width 1) (layer "B.Cu") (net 19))
 (segment (start 124.9 70.6) (end 128.9 74.6) (width 1) (layer "B.Cu") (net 19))
 (segment (start 117.3125 51.3875) (end 114.5 54.2) (width 1) (layer "B.Cu") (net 19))
 (segment (start 164.2 79.1) (end 165.8 80.7) (width 0.5) (layer "F.Cu") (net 1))
 (via (at 165.8 80.7) (size 0.6) (drill 0.3) (layers "F.Cu" "B.Cu") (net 1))
 (via (at 164.2 79.1) (size 0.6) (drill 0.3) (layers "F.Cu" "B.Cu") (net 1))
 (segment (start 166.5 81.4) (end 176.2 81.4) (width 0.5) (layer "B.Cu") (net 1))
 (segment (start 165.8 80.7) (end 166.5 81.4) (width 0.5) (layer "B.Cu") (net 1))
 (segment (start 154.28 78.8) (end 163.9 78.8) (width 0.5) (layer "B.Cu") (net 1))
 (segment (start 163.9 78.8) (end 164.2 79.1) (width 0.5) (layer "B.Cu") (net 1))
 (segment (start 172.38 61.02) (end 173.74 59.66) (width 0.5) (layer "B.Cu") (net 16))
 (segment (start 173.74 59.66) (end 176.3 59.66) (width 0.5) (layer "B.Cu") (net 16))
 (segment (start 169.52 61.02) (end 172.38 61.02) (width 0.5) (layer "B.Cu") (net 16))
 (segment (start 169.52 63.56) (end 171.74 63.56) (width 0.5) (layer "B.Cu") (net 17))
 (segment (start 173.1 62.2) (end 176.3 62.2) (width 0.5) (layer "B.Cu") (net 17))
 (segment (start 171.74 63.56) (end 173.1 62.2) (width 0.5) (layer "B.Cu") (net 17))
 (segment (start 177 52.75) (end 175.15 52.75) (width 0.5) (layer "F.Cu") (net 15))
 (segment (start 154.28 61.02) (end 166.08 61.02) (width 0.5) (layer "F.Cu") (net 15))
 (segment (start 175.15 52.75) (end 174.7 53.2) (width 0.5) (layer "F.Cu") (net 15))
 (segment (start 166.08 61.02) (end 166.1 61) (width 0.2) (layer "F.Cu") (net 15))
 (via (at 174.7 53.2) (size 0.6) (drill 0.3) (layers "F.Cu" "B.Cu") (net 15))
 (via (at 166.1 61) (size 0.6) (drill 0.3) (layers "F.Cu" "B.Cu") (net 15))
 (segment (start 166.1 61) (end 166.9 61) (width 0.5) (layer "B.Cu") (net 15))
 (segment (start 174.7 53.2) (end 176.3 54.8) (width 0.5) (layer "B.Cu") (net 15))
 (segment (start 174.02 57.12) (end 176.3 57.12) (width 0.5) (layer "B.Cu") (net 15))
 (segment (start 166.9 61) (end 168.1 59.8) (width 0.5) (layer "B.Cu") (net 15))
 (segment (start 174 57.1) (end 174.02 57.12) (width 0.2) (layer "B.Cu") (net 15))
 (segment (start 171.3 59.8) (end 174 57.1) (width 0.5) (layer "B.Cu") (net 15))
 (segment (start 168.1 59.8) (end 171.3 59.8) (width 0.5) (layer "B.Cu") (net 15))
 (segment (start 176.3 54.8) (end 176.3 57.12) (width 0.5) (layer "B.Cu") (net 15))
 (segment (start 171.5 51.45) (end 171.5 49.2) (width 0.5) (layer "F.Cu") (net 18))
 (segment (start 177 51.45) (end 177 49.1) (width 0.5) (layer "F.Cu") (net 12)))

